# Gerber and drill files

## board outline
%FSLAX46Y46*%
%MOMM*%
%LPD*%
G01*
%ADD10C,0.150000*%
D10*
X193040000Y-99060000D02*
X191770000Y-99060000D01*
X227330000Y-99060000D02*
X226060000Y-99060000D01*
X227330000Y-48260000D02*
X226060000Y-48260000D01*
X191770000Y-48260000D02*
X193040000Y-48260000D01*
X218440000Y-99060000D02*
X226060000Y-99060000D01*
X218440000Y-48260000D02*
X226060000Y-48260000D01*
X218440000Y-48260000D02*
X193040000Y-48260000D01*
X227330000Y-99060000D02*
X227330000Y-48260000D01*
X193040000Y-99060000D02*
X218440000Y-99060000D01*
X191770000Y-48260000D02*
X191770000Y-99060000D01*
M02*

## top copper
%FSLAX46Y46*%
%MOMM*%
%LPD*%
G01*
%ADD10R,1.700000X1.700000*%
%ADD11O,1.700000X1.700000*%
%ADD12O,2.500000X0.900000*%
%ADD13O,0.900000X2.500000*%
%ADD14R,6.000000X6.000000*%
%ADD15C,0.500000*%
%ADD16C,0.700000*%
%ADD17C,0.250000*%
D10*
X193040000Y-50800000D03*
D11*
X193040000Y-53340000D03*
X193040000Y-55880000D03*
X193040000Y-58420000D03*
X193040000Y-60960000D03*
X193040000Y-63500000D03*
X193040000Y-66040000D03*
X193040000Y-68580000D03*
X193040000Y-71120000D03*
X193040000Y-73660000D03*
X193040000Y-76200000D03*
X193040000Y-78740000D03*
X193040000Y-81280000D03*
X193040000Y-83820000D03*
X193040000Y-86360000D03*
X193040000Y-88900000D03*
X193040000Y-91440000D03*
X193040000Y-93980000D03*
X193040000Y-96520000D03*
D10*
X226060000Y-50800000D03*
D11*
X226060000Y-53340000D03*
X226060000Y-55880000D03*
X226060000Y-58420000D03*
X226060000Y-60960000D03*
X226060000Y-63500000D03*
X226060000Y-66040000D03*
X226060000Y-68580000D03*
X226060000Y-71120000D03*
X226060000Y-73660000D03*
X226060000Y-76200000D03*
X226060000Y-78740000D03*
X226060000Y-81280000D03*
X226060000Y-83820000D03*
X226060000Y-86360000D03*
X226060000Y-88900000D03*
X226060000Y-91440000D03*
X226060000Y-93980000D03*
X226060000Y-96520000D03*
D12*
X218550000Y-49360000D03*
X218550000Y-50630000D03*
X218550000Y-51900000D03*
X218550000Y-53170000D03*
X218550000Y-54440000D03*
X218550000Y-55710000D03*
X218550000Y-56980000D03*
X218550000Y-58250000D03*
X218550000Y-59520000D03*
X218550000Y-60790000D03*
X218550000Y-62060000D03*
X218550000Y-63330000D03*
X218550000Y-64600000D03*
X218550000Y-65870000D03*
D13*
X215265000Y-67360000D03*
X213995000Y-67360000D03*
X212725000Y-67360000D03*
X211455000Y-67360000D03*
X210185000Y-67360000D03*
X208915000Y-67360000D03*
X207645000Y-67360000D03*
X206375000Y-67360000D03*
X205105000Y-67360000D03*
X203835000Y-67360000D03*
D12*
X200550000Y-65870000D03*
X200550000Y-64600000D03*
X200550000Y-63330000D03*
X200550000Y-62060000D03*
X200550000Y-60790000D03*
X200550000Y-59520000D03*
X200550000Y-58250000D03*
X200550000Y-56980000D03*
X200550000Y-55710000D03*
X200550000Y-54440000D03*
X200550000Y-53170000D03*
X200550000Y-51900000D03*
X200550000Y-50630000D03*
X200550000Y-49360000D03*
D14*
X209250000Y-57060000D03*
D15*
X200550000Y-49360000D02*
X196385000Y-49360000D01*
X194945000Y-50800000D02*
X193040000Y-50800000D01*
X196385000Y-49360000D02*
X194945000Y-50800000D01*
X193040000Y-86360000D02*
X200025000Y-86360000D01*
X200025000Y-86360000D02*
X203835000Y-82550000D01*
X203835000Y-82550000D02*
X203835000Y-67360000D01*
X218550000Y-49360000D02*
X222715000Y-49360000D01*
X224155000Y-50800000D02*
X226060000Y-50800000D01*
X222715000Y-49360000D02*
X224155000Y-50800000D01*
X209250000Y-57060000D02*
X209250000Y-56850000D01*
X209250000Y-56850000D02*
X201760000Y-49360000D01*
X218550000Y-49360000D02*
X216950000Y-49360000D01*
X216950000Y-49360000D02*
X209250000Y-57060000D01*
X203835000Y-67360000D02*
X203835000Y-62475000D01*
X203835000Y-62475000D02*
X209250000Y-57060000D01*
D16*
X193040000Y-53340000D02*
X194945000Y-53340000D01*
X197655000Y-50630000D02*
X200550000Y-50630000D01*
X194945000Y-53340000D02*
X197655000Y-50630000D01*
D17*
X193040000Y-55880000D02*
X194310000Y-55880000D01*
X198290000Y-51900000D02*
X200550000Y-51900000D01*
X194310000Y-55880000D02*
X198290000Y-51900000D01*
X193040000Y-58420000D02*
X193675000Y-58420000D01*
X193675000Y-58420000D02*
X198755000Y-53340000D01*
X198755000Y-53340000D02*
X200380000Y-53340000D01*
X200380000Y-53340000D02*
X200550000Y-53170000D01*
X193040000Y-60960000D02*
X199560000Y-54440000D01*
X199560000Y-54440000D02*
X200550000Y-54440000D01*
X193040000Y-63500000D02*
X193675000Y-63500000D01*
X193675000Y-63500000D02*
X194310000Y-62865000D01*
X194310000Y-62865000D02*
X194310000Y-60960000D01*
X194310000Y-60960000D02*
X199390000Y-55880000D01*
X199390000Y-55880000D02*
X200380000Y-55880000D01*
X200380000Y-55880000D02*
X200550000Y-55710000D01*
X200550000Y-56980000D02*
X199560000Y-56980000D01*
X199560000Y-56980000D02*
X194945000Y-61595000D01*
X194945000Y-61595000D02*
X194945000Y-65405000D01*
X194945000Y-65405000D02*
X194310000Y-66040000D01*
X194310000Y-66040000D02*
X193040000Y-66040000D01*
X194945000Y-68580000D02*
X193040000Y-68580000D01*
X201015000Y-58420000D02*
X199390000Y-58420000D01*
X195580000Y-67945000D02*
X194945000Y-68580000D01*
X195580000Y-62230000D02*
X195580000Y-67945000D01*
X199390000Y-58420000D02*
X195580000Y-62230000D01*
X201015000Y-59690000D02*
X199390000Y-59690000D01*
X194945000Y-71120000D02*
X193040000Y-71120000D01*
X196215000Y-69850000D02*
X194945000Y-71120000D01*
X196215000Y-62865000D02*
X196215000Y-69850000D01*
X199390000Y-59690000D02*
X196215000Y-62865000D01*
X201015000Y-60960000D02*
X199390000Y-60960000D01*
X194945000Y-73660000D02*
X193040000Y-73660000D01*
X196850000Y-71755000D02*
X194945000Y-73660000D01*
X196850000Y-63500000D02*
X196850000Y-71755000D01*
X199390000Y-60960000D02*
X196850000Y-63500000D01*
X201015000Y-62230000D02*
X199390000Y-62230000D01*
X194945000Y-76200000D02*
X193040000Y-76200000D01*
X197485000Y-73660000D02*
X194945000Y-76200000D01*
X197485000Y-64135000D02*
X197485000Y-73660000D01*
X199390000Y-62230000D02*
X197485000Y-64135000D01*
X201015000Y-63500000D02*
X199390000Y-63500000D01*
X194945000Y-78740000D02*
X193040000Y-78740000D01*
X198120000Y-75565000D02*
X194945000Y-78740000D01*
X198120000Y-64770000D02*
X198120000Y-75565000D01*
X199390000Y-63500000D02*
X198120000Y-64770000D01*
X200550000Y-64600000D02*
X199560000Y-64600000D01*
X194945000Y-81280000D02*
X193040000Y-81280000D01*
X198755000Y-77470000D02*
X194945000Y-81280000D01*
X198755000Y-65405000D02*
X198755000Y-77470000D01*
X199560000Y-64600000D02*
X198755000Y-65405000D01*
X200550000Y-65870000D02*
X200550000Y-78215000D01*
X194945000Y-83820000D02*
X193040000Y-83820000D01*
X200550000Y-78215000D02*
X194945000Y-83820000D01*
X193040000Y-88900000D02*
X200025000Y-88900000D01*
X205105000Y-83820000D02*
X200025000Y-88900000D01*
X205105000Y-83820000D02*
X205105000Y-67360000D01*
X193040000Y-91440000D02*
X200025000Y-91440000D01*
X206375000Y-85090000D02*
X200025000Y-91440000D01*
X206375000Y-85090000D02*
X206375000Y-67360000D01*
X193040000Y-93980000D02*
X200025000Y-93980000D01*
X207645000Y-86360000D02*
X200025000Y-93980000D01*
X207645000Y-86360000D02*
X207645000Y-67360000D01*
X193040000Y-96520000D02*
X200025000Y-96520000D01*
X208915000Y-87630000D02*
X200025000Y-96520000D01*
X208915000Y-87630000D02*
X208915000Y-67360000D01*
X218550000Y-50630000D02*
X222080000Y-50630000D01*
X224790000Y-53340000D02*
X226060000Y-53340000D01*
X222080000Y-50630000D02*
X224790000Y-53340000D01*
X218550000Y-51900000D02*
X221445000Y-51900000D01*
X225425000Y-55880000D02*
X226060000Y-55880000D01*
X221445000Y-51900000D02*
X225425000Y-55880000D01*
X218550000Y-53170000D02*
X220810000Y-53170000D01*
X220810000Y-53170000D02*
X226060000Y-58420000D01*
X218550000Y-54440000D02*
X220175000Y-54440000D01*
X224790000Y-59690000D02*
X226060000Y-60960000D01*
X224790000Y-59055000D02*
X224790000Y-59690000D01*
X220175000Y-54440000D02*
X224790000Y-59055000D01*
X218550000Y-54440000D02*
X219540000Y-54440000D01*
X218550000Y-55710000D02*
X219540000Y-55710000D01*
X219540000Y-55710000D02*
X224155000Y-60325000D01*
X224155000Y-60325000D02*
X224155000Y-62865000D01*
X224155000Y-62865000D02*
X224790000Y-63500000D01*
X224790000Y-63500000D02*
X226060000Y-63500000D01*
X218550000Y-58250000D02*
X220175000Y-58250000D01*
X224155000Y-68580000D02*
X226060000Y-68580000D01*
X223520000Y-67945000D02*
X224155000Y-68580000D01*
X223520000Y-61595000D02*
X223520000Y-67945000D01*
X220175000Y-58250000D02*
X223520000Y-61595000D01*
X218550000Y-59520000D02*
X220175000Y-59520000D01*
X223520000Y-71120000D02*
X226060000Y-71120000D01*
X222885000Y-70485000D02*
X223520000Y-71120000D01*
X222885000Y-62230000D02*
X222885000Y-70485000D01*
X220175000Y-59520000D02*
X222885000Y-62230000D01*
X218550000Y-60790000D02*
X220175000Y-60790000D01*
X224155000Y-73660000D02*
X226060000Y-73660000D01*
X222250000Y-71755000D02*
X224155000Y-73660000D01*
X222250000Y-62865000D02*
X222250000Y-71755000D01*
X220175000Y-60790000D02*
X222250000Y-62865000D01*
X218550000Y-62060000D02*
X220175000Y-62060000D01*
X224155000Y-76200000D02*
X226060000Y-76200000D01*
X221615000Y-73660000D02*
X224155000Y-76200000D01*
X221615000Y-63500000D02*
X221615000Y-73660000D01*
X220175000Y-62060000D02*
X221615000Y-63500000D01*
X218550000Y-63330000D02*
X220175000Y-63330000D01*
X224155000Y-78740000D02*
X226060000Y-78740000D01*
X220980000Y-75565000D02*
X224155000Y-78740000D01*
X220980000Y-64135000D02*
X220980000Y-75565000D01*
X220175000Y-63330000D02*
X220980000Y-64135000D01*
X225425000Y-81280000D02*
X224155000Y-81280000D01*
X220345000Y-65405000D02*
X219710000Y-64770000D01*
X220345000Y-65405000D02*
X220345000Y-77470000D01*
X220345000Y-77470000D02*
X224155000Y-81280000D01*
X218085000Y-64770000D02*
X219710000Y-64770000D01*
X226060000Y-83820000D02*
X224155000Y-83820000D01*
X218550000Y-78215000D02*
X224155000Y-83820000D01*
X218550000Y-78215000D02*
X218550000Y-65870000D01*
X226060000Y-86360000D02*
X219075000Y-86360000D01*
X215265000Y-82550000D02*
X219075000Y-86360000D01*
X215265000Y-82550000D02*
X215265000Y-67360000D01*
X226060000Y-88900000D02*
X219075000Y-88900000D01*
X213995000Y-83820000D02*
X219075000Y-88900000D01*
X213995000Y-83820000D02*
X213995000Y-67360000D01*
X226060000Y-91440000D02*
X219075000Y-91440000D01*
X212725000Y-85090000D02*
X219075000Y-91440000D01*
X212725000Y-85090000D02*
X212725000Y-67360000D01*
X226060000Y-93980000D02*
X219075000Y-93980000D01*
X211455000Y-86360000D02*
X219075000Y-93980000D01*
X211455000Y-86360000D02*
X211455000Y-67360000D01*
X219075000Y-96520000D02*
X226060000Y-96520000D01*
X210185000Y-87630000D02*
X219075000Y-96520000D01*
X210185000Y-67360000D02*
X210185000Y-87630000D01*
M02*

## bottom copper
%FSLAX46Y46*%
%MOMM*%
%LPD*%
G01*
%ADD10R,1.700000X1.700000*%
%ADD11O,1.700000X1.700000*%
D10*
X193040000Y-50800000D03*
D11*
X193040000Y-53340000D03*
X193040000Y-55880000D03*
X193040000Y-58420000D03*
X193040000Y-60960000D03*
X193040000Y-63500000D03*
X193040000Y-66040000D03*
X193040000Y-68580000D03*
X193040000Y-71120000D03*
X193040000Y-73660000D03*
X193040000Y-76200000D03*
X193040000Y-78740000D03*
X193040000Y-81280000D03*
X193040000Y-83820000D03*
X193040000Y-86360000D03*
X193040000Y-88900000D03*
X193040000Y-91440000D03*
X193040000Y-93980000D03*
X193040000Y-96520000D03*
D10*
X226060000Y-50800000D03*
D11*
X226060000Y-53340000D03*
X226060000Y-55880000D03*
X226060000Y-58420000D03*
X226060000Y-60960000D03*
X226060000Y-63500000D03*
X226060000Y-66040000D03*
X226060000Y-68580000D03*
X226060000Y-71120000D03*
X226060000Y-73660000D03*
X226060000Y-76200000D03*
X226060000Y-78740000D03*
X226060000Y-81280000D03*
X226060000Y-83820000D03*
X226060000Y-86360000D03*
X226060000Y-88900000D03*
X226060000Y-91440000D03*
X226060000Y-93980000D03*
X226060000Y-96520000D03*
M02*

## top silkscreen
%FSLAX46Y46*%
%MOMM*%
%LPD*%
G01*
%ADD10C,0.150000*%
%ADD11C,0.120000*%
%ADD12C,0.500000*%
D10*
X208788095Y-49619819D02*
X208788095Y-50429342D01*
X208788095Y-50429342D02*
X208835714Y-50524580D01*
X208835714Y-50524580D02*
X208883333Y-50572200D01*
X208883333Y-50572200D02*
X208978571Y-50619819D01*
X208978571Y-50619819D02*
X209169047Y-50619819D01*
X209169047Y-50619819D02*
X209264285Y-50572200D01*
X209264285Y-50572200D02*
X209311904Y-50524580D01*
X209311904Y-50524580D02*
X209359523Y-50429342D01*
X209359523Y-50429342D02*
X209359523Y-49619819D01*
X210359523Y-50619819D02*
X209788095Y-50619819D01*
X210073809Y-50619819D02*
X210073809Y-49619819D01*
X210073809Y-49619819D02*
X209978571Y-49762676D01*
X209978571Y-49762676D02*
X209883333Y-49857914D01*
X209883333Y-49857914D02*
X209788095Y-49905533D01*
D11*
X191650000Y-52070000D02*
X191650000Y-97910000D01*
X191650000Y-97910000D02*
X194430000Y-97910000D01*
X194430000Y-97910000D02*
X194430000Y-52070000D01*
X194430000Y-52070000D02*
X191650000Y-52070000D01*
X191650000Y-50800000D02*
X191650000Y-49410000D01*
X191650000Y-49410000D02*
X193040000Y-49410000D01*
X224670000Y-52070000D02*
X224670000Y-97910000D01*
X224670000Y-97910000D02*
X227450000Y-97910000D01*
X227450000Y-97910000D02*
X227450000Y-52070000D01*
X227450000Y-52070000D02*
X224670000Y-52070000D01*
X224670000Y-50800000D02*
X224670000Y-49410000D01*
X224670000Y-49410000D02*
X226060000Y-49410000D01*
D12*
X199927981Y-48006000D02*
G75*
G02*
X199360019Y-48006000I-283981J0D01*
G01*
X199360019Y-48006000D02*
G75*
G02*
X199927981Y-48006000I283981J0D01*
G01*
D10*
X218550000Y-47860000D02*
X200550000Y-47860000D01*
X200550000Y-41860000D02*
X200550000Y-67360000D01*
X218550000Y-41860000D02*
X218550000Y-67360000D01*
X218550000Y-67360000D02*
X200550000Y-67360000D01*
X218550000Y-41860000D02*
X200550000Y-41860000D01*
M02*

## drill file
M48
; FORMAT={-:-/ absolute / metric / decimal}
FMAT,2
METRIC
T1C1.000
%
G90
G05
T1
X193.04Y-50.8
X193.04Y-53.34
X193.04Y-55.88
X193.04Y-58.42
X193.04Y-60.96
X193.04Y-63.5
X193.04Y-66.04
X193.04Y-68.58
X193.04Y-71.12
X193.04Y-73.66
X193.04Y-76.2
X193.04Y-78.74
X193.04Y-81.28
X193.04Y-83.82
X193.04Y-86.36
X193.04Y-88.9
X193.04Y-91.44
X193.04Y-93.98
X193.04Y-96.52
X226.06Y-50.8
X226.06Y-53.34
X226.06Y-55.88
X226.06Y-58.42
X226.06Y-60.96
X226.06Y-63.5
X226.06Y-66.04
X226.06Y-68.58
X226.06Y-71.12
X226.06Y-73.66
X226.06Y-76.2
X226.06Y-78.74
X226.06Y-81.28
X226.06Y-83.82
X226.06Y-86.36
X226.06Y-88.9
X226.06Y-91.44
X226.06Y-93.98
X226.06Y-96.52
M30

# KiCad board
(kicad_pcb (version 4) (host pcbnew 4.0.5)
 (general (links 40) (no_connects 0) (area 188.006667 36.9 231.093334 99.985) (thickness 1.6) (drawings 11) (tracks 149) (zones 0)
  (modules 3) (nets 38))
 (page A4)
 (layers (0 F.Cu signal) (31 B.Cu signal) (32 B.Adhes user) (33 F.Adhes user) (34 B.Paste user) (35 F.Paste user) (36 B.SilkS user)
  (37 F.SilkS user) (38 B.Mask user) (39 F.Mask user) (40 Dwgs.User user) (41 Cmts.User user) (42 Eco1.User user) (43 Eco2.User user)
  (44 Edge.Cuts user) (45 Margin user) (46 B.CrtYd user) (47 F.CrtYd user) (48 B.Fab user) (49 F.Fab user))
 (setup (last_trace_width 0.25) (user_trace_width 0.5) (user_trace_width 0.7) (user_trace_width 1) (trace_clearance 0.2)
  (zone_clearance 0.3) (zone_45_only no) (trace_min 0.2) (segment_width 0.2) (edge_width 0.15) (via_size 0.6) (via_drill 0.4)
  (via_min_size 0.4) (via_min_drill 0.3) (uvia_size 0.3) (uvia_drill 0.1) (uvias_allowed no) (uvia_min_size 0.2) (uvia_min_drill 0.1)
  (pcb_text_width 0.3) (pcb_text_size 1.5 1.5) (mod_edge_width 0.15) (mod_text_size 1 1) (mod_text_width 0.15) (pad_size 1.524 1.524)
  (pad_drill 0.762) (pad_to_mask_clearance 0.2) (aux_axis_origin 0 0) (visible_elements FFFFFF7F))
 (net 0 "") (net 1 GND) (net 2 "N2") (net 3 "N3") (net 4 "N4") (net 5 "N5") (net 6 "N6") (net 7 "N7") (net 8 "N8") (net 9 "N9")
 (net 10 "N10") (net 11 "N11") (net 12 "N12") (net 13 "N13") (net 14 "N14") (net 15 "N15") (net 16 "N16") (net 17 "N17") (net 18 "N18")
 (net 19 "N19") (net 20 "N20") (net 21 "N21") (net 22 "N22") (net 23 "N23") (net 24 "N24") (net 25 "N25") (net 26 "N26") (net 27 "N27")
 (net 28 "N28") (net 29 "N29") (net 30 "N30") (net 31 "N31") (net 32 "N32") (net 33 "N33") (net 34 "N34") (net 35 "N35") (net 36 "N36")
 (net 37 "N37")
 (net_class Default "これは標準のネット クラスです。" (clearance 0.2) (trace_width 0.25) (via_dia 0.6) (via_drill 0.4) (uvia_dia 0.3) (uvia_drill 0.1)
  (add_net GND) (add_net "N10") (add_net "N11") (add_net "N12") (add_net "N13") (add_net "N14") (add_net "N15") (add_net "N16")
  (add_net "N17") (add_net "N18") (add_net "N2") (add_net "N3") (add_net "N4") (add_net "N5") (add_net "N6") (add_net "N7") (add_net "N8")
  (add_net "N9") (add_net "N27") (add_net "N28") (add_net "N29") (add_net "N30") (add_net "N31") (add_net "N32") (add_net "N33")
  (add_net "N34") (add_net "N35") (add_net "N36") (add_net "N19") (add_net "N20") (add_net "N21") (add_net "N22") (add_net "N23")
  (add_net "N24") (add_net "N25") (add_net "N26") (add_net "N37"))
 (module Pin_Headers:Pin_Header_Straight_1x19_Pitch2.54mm (layer F.Cu) (at 193.04 50.8)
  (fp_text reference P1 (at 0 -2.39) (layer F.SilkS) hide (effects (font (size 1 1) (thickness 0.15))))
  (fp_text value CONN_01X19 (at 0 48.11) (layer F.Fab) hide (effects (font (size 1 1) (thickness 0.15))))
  (fp_line (start -1.39 1.27) (end -1.39 47.11) (layer F.SilkS) (width 0.12))
  (fp_line (start -1.39 47.11) (end 1.39 47.11) (layer F.SilkS) (width 0.12))
  (fp_line (start 1.39 47.11) (end 1.39 1.27) (layer F.SilkS) (width 0.12))
  (fp_line (start 1.39 1.27) (end -1.39 1.27) (layer F.SilkS) (width 0.12))
  (fp_line (start -1.39 0) (end -1.39 -1.39) (layer F.SilkS) (width 0.12))
  (fp_line (start -1.39 -1.39) (end 0 -1.39) (layer F.SilkS) (width 0.12))
  (pad 1 thru_hole rect (at 0 0) (size 1.7 1.7) (drill 1) (layers *.Cu *.Mask) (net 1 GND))
  (pad 2 thru_hole oval (at 0 2.54) (size 1.7 1.7) (drill 1) (layers *.Cu *.Mask) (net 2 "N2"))
  (pad 3 thru_hole oval (at 0 5.08) (size 1.7 1.7) (drill 1) (layers *.Cu *.Mask) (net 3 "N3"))
  (pad 4 thru_hole oval (at 0 7.62) (size 1.7 1.7) (drill 1) (layers *.Cu *.Mask) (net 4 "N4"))
  (pad 5 thru_hole oval (at 0 10.16) (size 1.7 1.7) (drill 1) (layers *.Cu *.Mask) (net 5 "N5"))
  (pad 6 thru_hole oval (at 0 12.7) (size 1.7 1.7) (drill 1) (layers *.Cu *.Mask) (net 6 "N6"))
  (pad 7 thru_hole oval (at 0 15.24) (size 1.7 1.7) (drill 1) (layers *.Cu *.Mask) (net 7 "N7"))
  (pad 8 thru_hole oval (at 0 17.78) (size 1.7 1.7) (drill 1) (layers *.Cu *.Mask) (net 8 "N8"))
  (pad 9 thru_hole oval (at 0 20.32) (size 1.7 1.7) (drill 1) (layers *.Cu *.Mask) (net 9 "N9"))
  (pad 10 thru_hole oval (at 0 22.86) (size 1.7 1.7) (drill 1) (layers *.Cu *.Mask) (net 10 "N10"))
  (pad 11 thru_hole oval (at 0 25.4) (size 1.7 1.7) (drill 1) (layers *.Cu *.Mask) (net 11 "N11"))
  (pad 12 thru_hole oval (at 0 27.94) (size 1.7 1.7) (drill 1) (layers *.Cu *.Mask) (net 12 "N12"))
  (pad 13 thru_hole oval (at 0 30.48) (size 1.7 1.7) (drill 1) (layers *.Cu *.Mask) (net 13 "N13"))
  (pad 14 thru_hole oval (at 0 33.02) (size 1.7 1.7) (drill 1) (layers *.Cu *.Mask) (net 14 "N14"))
  (pad 15 thru_hole oval (at 0 35.56) (size 1.7 1.7) (drill 1) (layers *.Cu *.Mask) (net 1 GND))
  (pad 16 thru_hole oval (at 0 38.1) (size 1.7 1.7) (drill 1) (layers *.Cu *.Mask) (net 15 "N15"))
  (pad 17 thru_hole oval (at 0 40.64) (size 1.7 1.7) (drill 1) (layers *.Cu *.Mask) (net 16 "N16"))
  (pad 18 thru_hole oval (at 0 43.18) (size 1.7 1.7) (drill 1) (layers *.Cu *.Mask) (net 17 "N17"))
  (pad 19 thru_hole oval (at 0 45.72) (size 1.7 1.7) (drill 1) (layers *.Cu *.Mask) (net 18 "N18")))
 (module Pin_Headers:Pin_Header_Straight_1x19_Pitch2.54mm (layer F.Cu) (at 226.06 50.8)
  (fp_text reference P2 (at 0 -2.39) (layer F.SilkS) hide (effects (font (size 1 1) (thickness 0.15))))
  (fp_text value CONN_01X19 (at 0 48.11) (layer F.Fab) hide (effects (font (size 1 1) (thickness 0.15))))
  (fp_line (start -1.39 1.27) (end -1.39 47.11) (layer F.SilkS) (width 0.12))
  (fp_line (start -1.39 47.11) (end 1.39 47.11) (layer F.SilkS) (width 0.12))
  (fp_line (start 1.39 47.11) (end 1.39 1.27) (layer F.SilkS) (width 0.12))
  (fp_line (start 1.39 1.27) (end -1.39 1.27) (layer F.SilkS) (width 0.12))
  (fp_line (start -1.39 0) (end -1.39 -1.39) (layer F.SilkS) (width 0.12))
  (fp_line (start -1.39 -1.39) (end 0 -1.39) (layer F.SilkS) (width 0.12))
  (pad 1 thru_hole rect (at 0 0) (size 1.7 1.7) (drill 1) (layers *.Cu *.Mask) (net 1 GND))
  (pad 2 thru_hole oval (at 0 2.54) (size 1.7 1.7) (drill 1) (layers *.Cu *.Mask) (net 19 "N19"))
  (pad 3 thru_hole oval (at 0 5.08) (size 1.7 1.7) (drill 1) (layers *.Cu *.Mask) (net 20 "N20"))
  (pad 4 thru_hole oval (at 0 7.62) (size 1.7 1.7) (drill 1) (layers *.Cu *.Mask) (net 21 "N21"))
  (pad 5 thru_hole oval (at 0 10.16) (size 1.7 1.7) (drill 1) (layers *.Cu *.Mask) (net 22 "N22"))
  (pad 6 thru_hole oval (at 0 12.7) (size 1.7 1.7) (drill 1) (layers *.Cu *.Mask) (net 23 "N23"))
  (pad 7 thru_hole oval (at 0 15.24) (size 1.7 1.7) (drill 1) (layers *.Cu *.Mask) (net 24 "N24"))
  (pad 8 thru_hole oval (at 0 17.78) (size 1.7 1.7) (drill 1) (layers *.Cu *.Mask) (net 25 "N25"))
  (pad 9 thru_hole oval (at 0 20.32) (size 1.7 1.7) (drill 1) (layers *.Cu *.Mask) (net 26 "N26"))
  (pad 10 thru_hole oval (at 0 22.86) (size 1.7 1.7) (drill 1) (layers *.Cu *.Mask) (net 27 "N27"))
  (pad 11 thru_hole oval (at 0 25.4) (size 1.7 1.7) (drill 1) (layers *.Cu *.Mask) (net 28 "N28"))
  (pad 12 thru_hole oval (at 0 27.94) (size 1.7 1.7) (drill 1) (layers *.Cu *.Mask) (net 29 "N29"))
  (pad 13 thru_hole oval (at 0 30.48) (size 1.7 1.7) (drill 1) (layers *.Cu *.Mask) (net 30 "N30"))
  (pad 14 thru_hole oval (at 0 33.02) (size 1.7 1.7) (drill 1) (layers *.Cu *.Mask) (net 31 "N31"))
  (pad 15 thru_hole oval (at 0 35.56) (size 1.7 1.7) (drill 1) (layers *.Cu *.Mask) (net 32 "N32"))
  (pad 16 thru_hole oval (at 0 38.1) (size 1.7 1.7) (drill 1) (layers *.Cu *.Mask) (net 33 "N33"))
  (pad 17 thru_hole oval (at 0 40.64) (size 1.7 1.7) (drill 1) (layers *.Cu *.Mask) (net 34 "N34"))
  (pad 18 thru_hole oval (at 0 43.18) (size 1.7 1.7) (drill 1) (layers *.Cu *.Mask) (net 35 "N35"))
  (pad 19 thru_hole oval (at 0 45.72) (size 1.7 1.7) (drill 1) (layers *.Cu *.Mask) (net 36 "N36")))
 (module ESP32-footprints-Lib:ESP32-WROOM (layer F.Cu) (at 209.55 54.61 180)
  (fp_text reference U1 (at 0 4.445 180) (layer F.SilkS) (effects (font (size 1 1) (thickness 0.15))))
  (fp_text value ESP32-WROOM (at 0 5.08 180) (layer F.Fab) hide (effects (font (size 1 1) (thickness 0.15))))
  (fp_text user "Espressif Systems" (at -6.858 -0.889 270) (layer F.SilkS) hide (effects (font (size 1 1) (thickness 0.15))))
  (fp_circle (center 9.906 6.604) (end 10.033 6.858) (layer F.SilkS) (width 0.5))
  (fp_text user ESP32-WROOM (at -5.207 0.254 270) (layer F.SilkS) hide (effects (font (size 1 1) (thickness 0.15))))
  (fp_line (start -9 6.75) (end 9 6.75) (layer F.SilkS) (width 0.15))
  (fp_line (start 9 12.75) (end 9 -12.75) (layer F.SilkS) (width 0.15))
  (fp_line (start -9 12.75) (end -9 -12.75) (layer F.SilkS) (width 0.15))
  (fp_line (start -9 -12.75) (end 9 -12.75) (layer F.SilkS) (width 0.15))
  (fp_line (start -9 12.75) (end 9 12.75) (layer F.SilkS) (width 0.15))
  (pad 38 smd oval (at -9 5.25 180) (size 2.5 0.9) (layers F.Cu F.Paste F.Mask) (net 1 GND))
  (pad 37 smd oval (at -9 3.98 180) (size 2.5 0.9) (layers F.Cu F.Paste F.Mask) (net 19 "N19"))
  (pad 36 smd oval (at -9 2.71 180) (size 2.5 0.9) (layers F.Cu F.Paste F.Mask) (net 20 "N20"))
  (pad 35 smd oval (at -9 1.44 180) (size 2.5 0.9) (layers F.Cu F.Paste F.Mask) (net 21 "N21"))
  (pad 34 smd oval (at -9 0.17 180) (size 2.5 0.9) (layers F.Cu F.Paste F.Mask) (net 22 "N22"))
  (pad 33 smd oval (at -9 -1.1 180) (size 2.5 0.9) (layers F.Cu F.Paste F.Mask) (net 23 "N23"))
  (pad 32 smd oval (at -9 -2.37 180) (size 2.5 0.9) (layers F.Cu F.Paste F.Mask) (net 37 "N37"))
  (pad 31 smd oval (at -9 -3.64 180) (size 2.5 0.9) (layers F.Cu F.Paste F.Mask) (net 25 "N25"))
  (pad 30 smd oval (at -9 -4.91 180) (size 2.5 0.9) (layers F.Cu F.Paste F.Mask) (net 26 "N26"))
  (pad 29 smd oval (at -9 -6.18 180) (size 2.5 0.9) (layers F.Cu F.Paste F.Mask) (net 27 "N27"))
  (pad 28 smd oval (at -9 -7.45 180) (size 2.5 0.9) (layers F.Cu F.Paste F.Mask) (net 28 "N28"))
  (pad 27 smd oval (at -9 -8.72 180) (size 2.5 0.9) (layers F.Cu F.Paste F.Mask) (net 29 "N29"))
  (pad 26 smd oval (at -9 -9.99 180) (size 2.5 0.9) (layers F.Cu F.Paste F.Mask) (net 30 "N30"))
  (pad 25 smd oval (at -9 -11.26 180) (size 2.5 0.9) (layers F.Cu F.Paste F.Mask) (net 31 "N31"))
  (pad 24 smd oval (at -5.715 -12.75 180) (size 0.9 2.5) (layers F.Cu F.Paste F.Mask) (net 32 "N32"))
  (pad 23 smd oval (at -4.445 -12.75 180) (size 0.9 2.5) (layers F.Cu F.Paste F.Mask) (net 33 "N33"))
  (pad 22 smd oval (at -3.175 -12.75 180) (size 0.9 2.5) (layers F.Cu F.Paste F.Mask) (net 34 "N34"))
  (pad 21 smd oval (at -1.905 -12.75 180) (size 0.9 2.5) (layers F.Cu F.Paste F.Mask) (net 35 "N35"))
  (pad 20 smd oval (at -0.635 -12.75 180) (size 0.9 2.5) (layers F.Cu F.Paste F.Mask) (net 36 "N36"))
  (pad 19 smd oval (at 0.635 -12.75 180) (size 0.9 2.5) (layers F.Cu F.Paste F.Mask) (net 18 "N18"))
  (pad 18 smd oval (at 1.905 -12.75 180) (size 0.9 2.5) (layers F.Cu F.Paste F.Mask) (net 17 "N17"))
  (pad 17 smd oval (at 3.175 -12.75 180) (size 0.9 2.5) (layers F.Cu F.Paste F.Mask) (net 16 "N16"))
  (pad 16 smd oval (at 4.445 -12.75 180) (size 0.9 2.5) (layers F.Cu F.Paste F.Mask) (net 15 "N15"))
  (pad 15 smd oval (at 5.715 -12.75 180) (size 0.9 2.5) (layers F.Cu F.Paste F.Mask) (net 1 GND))
  (pad 14 smd oval (at 9 -11.26 180) (size 2.5 0.9) (layers F.Cu F.Paste F.Mask) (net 14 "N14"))
  (pad 13 smd oval (at 9 -9.99 180) (size 2.5 0.9) (layers F.Cu F.Paste F.Mask) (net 13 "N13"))
  (pad 12 smd oval (at 9 -8.72 180) (size 2.5 0.9) (layers F.Cu F.Paste F.Mask) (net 12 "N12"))
  (pad 11 smd oval (at 9 -7.45 180) (size 2.5 0.9) (layers F.Cu F.Paste F.Mask) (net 11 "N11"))
  (pad 10 smd oval (at 9 -6.18 180) (size 2.5 0.9) (layers F.Cu F.Paste F.Mask) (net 10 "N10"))
  (pad 9 smd oval (at 9 -4.91 180) (size 2.5 0.9) (layers F.Cu F.Paste F.Mask) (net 9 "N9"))
  (pad 8 smd oval (at 9 -3.64 180) (size 2.5 0.9) (layers F.Cu F.Paste F.Mask) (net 8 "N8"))
  (pad 7 smd oval (at 9 -2.37 180) (size 2.5 0.9) (layers F.Cu F.Paste F.Mask) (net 7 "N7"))
  (pad 6 smd oval (at 9 -1.1 180) (size 2.5 0.9) (layers F.Cu F.Paste F.Mask) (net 6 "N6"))
  (pad 5 smd oval (at 9 0.17 180) (size 2.5 0.9) (layers F.Cu F.Paste F.Mask) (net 5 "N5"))
  (pad 4 smd oval (at 9 1.44 180) (size 2.5 0.9) (layers F.Cu F.Paste F.Mask) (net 4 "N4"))
  (pad 3 smd oval (at 9 2.71 180) (size 2.5 0.9) (layers F.Cu F.Paste F.Mask) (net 3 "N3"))
  (pad 2 smd oval (at 9 3.98 180) (size 2.5 0.9) (layers F.Cu F.Paste F.Mask) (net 2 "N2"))
  (pad 1 smd oval (at 9 5.25 180) (size 2.5 0.9) (layers F.Cu F.Paste F.Mask) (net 1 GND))
  (pad 39 smd rect (at 0.3 -2.45 180) (size 6 6) (layers F.Cu F.Paste F.Mask) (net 1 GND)))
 (gr_line (start 193.04 99.06) (end 191.77 99.06) (angle 90) (layer Edge.Cuts) (width 0.15))
 (gr_line (start 227.33 99.06) (end 226.06 99.06) (angle 90) (layer Edge.Cuts) (width 0.15))
 (gr_line (start 227.33 48.26) (end 226.06 48.26) (angle 90) (layer Edge.Cuts) (width 0.15))
 (gr_line (start 191.77 48.26) (end 193.04 48.26) (angle 90) (layer Edge.Cuts) (width 0.15))
 (gr_line (start 218.44 99.06) (end 226.06 99.06) (angle 90) (layer Edge.Cuts) (width 0.15))
 (gr_line (start 218.44 48.26) (end 226.06 48.26) (angle 90) (layer Edge.Cuts) (width 0.15))
 (gr_line (start 218.44 48.26) (end 193.04 48.26) (angle 90) (layer Edge.Cuts) (width 0.15))
 (gr_line (start 227.33 99.06) (end 227.33 48.26) (angle 90) (layer Edge.Cuts) (width 0.15))
 (gr_line (start 193.04 99.06) (end 218.44 99.06) (angle 90) (layer Edge.Cuts) (width 0.15))
 (gr_line (start 191.77 48.26) (end 191.77 99.06) (angle 90) (layer Edge.Cuts) (width 0.15))
 (segment (start 200.55 49.36) (end 196.385 49.36) (width 0.5) (layer F.Cu) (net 1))
 (segment (start 194.945 50.8) (end 193.04 50.8) (width 0.5) (layer F.Cu) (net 1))
 (segment (start 196.385 49.36) (end 194.945 50.8) (width 0.5) (layer F.Cu) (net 1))
 (segment (start 193.04 86.36) (end 200.025 86.36) (width 0.5) (layer F.Cu) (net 1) (status 10))
 (segment (start 200.025 86.36) (end 203.835 82.55) (width 0.5) (layer F.Cu) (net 1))
 (segment (start 203.835 82.55) (end 203.835 67.36) (width 0.5) (layer F.Cu) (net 1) (status 20))
 (segment (start 218.55 49.36) (end 222.715 49.36) (width 0.5) (layer F.Cu) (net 1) (status 10))
 (segment (start 224.155 50.8) (end 226.06 50.8) (width 0.5) (layer F.Cu) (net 1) (status 20))
 (segment (start 222.715 49.36) (end 224.155 50.8) (width 0.5) (layer F.Cu) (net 1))
 (segment (start 209.25 57.06) (end 209.25 56.85) (width 0.5) (layer F.Cu) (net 1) (status 30))
 (segment (start 209.25 56.85) (end 201.76 49.36) (width 0.5) (layer F.Cu) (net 1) (status 30))
 (segment (start 218.55 49.36) (end 216.95 49.36) (width 0.5) (layer F.Cu) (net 1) (status 10))
 (segment (start 216.95 49.36) (end 209.25 57.06) (width 0.5) (layer F.Cu) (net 1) (status 20))
 (segment (start 203.835 67.36) (end 203.835 62.475) (width 0.5) (layer F.Cu) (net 1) (status 10))
 (segment (start 203.835 62.475) (end 209.25 57.06) (width 0.5) (layer F.Cu) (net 1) (status 20))
 (segment (start 193.04 53.34) (end 194.945 53.34) (width 0.7) (layer F.Cu) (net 2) (status 10))
 (segment (start 197.655 50.63) (end 200.55 50.63) (width 0.7) (layer F.Cu) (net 2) (status 20))
 (segment (start 194.945 53.34) (end 197.655 50.63) (width 0.7) (layer F.Cu) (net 2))
 (segment (start 193.04 55.88) (end 194.31 55.88) (width 0.25) (layer F.Cu) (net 3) (status 10))
 (segment (start 198.29 51.9) (end 200.55 51.9) (width 0.25) (layer F.Cu) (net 3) (status 20))
 (segment (start 194.31 55.88) (end 198.29 51.9) (width 0.25) (layer F.Cu) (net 3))
 (segment (start 193.04 58.42) (end 193.675 58.42) (width 0.25) (layer F.Cu) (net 4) (status 30))
 (segment (start 193.675 58.42) (end 198.755 53.34) (width 0.25) (layer F.Cu) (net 4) (status 10))
 (segment (start 198.755 53.34) (end 200.38 53.34) (width 0.25) (layer F.Cu) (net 4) (status 20))
 (segment (start 200.38 53.34) (end 200.55 53.17) (width 0.25) (layer F.Cu) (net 4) (status 30))
 (segment (start 193.04 60.96) (end 199.56 54.44) (width 0.25) (layer F.Cu) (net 5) (status 30))
 (segment (start 199.56 54.44) (end 200.55 54.44) (width 0.25) (layer F.Cu) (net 5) (status 30))
 (segment (start 193.04 63.5) (end 193.675 63.5) (width 0.25) (layer F.Cu) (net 6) (status 30))
 (segment (start 193.675 63.5) (end 194.31 62.865) (width 0.25) (layer F.Cu) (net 6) (status 10))
 (segment (start 194.31 62.865) (end 194.31 60.96) (width 0.25) (layer F.Cu) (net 6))
 (segment (start 194.31 60.96) (end 199.39 55.88) (width 0.25) (layer F.Cu) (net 6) (status 20))
 (segment (start 199.39 55.88) (end 200.38 55.88) (width 0.25) (layer F.Cu) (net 6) (status 30))
 (segment (start 200.38 55.88) (end 200.55 55.71) (width 0.25) (layer F.Cu) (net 6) (status 30))
 (segment (start 200.55 56.98) (end 199.56 56.98) (width 0.25) (layer F.Cu) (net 7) (status 30))
 (segment (start 199.56 56.98) (end 194.945 61.595) (width 0.25) (layer F.Cu) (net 7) (status 10))
 (segment (start 194.945 61.595) (end 194.945 65.405) (width 0.25) (layer F.Cu) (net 7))
 (segment (start 194.945 65.405) (end 194.31 66.04) (width 0.25) (layer F.Cu) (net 7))
 (segment (start 194.31 66.04) (end 193.04 66.04) (width 0.25) (layer F.Cu) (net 7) (status 20))
 (segment (start 194.945 68.58) (end 193.04 68.58) (width 0.25) (layer F.Cu) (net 8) (status 20))
 (segment (start 201.015 58.42) (end 199.39 58.42) (width 0.25) (layer F.Cu) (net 8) (status 30))
 (segment (start 195.58 67.945) (end 194.945 68.58) (width 0.25) (layer F.Cu) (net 8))
 (segment (start 195.58 62.23) (end 195.58 67.945) (width 0.25) (layer F.Cu) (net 8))
 (segment (start 199.39 58.42) (end 195.58 62.23) (width 0.25) (layer F.Cu) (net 8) (status 10))
 (segment (start 201.015 59.69) (end 199.39 59.69) (width 0.25) (layer F.Cu) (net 9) (status 30))
 (segment (start 194.945 71.12) (end 193.04 71.12) (width 0.25) (layer F.Cu) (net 9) (status 20))
 (segment (start 196.215 69.85) (end 194.945 71.12) (width 0.25) (layer F.Cu) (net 9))
 (segment (start 196.215 62.865) (end 196.215 69.85) (width 0.25) (layer F.Cu) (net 9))
 (segment (start 199.39 59.69) (end 196.215 62.865) (width 0.25) (layer F.Cu) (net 9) (status 10))
 (segment (start 201.015 60.96) (end 199.39 60.96) (width 0.25) (layer F.Cu) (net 10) (status 30))
 (segment (start 194.945 73.66) (end 193.04 73.66) (width 0.25) (layer F.Cu) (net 10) (status 20))
 (segment (start 196.85 71.755) (end 194.945 73.66) (width 0.25) (layer F.Cu) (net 10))
 (segment (start 196.85 63.5) (end 196.85 71.755) (width 0.25) (layer F.Cu) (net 10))
 (segment (start 199.39 60.96) (end 196.85 63.5) (width 0.25) (layer F.Cu) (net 10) (status 10))
 (segment (start 201.015 62.23) (end 199.39 62.23) (width 0.25) (layer F.Cu) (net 11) (status 30))
 (segment (start 194.945 76.2) (end 193.04 76.2) (width 0.25) (layer F.Cu) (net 11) (status 20))
 (segment (start 197.485 73.66) (end 194.945 76.2) (width 0.25) (layer F.Cu) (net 11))
 (segment (start 197.485 64.135) (end 197.485 73.66) (width 0.25) (layer F.Cu) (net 11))
 (segment (start 199.39 62.23) (end 197.485 64.135) (width 0.25) (layer F.Cu) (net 11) (status 10))
 (segment (start 201.015 63.5) (end 199.39 63.5) (width 0.25) (layer F.Cu) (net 12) (status 30))
 (segment (start 194.945 78.74) (end 193.04 78.74) (width 0.25) (layer F.Cu) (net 12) (status 20))
 (segment (start 198.12 75.565) (end 194.945 78.74) (width 0.25) (layer F.Cu) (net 12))
 (segment (start 198.12 64.77) (end 198.12 75.565) (width 0.25) (layer F.Cu) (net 12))
 (segment (start 199.39 63.5) (end 198.12 64.77) (width 0.25) (layer F.Cu) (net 12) (status 10))
 (segment (start 200.55 64.6) (end 199.56 64.6) (width 0.25) (layer F.Cu) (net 13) (status 30))
 (segment (start 194.945 81.28) (end 193.04 81.28) (width 0.25) (layer F.Cu) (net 13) (status 20))
 (segment (start 198.755 77.47) (end 194.945 81.28) (width 0.25) (layer F.Cu) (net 13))
 (segment (start 198.755 65.405) (end 198.755 77.47) (width 0.25) (layer F.Cu) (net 13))
 (segment (start 199.56 64.6) (end 198.755 65.405) (width 0.25) (layer F.Cu) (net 13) (status 10))
 (segment (start 200.55 65.87) (end 200.55 78.215) (width 0.25) (layer F.Cu) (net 14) (status 10))
 (segment (start 194.945 83.82) (end 193.04 83.82) (width 0.25) (layer F.Cu) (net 14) (status 20))
 (segment (start 200.55 78.215) (end 194.945 83.82) (width 0.25) (layer F.Cu) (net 14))
 (segment (start 193.04 88.9) (end 200.025 88.9) (width 0.25) (layer F.Cu) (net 15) (status 10))
 (segment (start 205.105 83.82) (end 200.025 88.9) (width 0.25) (layer F.Cu) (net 15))
 (segment (start 205.105 83.82) (end 205.105 67.36) (width 0.25) (layer F.Cu) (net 15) (status 20))
 (segment (start 193.04 91.44) (end 200.025 91.44) (width 0.25) (layer F.Cu) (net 16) (status 10))
 (segment (start 206.375 85.09) (end 200.025 91.44) (width 0.25) (layer F.Cu) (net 16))
 (segment (start 206.375 85.09) (end 206.375 67.36) (width 0.25) (layer F.Cu) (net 16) (status 20))
 (segment (start 193.04 93.98) (end 200.025 93.98) (width 0.25) (layer F.Cu) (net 17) (status 10))
 (segment (start 207.645 86.36) (end 200.025 93.98) (width 0.25) (layer F.Cu) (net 17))
 (segment (start 207.645 86.36) (end 207.645 67.36) (width 0.25) (layer F.Cu) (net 17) (status 20))
 (segment (start 193.04 96.52) (end 200.025 96.52) (width 0.25) (layer F.Cu) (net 18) (status 10))
 (segment (start 208.915 87.63) (end 200.025 96.52) (width 0.25) (layer F.Cu) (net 18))
 (segment (start 208.915 87.63) (end 208.915 67.36) (width 0.25) (layer F.Cu) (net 18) (status 20))
 (segment (start 218.55 50.63) (end 222.08 50.63) (width 0.25) (layer F.Cu) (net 19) (status 10))
 (segment (start 224.79 53.34) (end 226.06 53.34) (width 0.25) (layer F.Cu) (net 19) (status 20))
 (segment (start 222.08 50.63) (end 224.79 53.34) (width 0.25) (layer F.Cu) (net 19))
 (segment (start 218.55 51.9) (end 221.445 51.9) (width 0.25) (layer F.Cu) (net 20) (status 10))
 (segment (start 225.425 55.88) (end 226.06 55.88) (width 0.25) (layer F.Cu) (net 20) (status 30))
 (segment (start 221.445 51.9) (end 225.425 55.88) (width 0.25) (layer F.Cu) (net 20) (status 20))
 (segment (start 218.55 53.17) (end 220.81 53.17) (width 0.25) (layer F.Cu) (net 21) (status 10))
 (segment (start 220.81 53.17) (end 226.06 58.42) (width 0.25) (layer F.Cu) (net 21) (status 20))
 (segment (start 218.55 54.44) (end 220.175 54.44) (width 0.25) (layer F.Cu) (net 22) (status 10))
 (segment (start 224.79 59.69) (end 226.06 60.96) (width 0.25) (layer F.Cu) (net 22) (status 20))
 (segment (start 224.79 59.055) (end 224.79 59.69) (width 0.25) (layer F.Cu) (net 22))
 (segment (start 220.175 54.44) (end 224.79 59.055) (width 0.25) (layer F.Cu) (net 22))
 (segment (start 218.55 54.44) (end 219.54 54.44) (width 0.25) (layer F.Cu) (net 22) (status 30))
 (segment (start 218.55 55.71) (end 219.54 55.71) (width 0.25) (layer F.Cu) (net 23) (status 30))
 (segment (start 219.54 55.71) (end 224.155 60.325) (width 0.25) (layer F.Cu) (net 23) (status 10))
 (segment (start 224.155 60.325) (end 224.155 62.865) (width 0.25) (layer F.Cu) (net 23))
 (segment (start 224.155 62.865) (end 224.79 63.5) (width 0.25) (layer F.Cu) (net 23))
 (segment (start 224.79 63.5) (end 226.06 63.5) (width 0.25) (layer F.Cu) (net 23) (status 20))
 (segment (start 218.55 58.25) (end 220.175 58.25) (width 0.25) (layer F.Cu) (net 25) (status 10))
 (segment (start 224.155 68.58) (end 226.06 68.58) (width 0.25) (layer F.Cu) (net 25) (status 20))
 (segment (start 223.52 67.945) (end 224.155 68.58) (width 0.25) (layer F.Cu) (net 25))
 (segment (start 223.52 61.595) (end 223.52 67.945) (width 0.25) (layer F.Cu) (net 25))
 (segment (start 220.175 58.25) (end 223.52 61.595) (width 0.25) (layer F.Cu) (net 25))
 (segment (start 218.55 59.52) (end 220.175 59.52) (width 0.25) (layer F.Cu) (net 26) (status 10))
 (segment (start 223.52 71.12) (end 226.06 71.12) (width 0.25) (layer F.Cu) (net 26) (status 20))
 (segment (start 222.885 70.485) (end 223.52 71.12) (width 0.25) (layer F.Cu) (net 26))
 (segment (start 222.885 62.23) (end 222.885 70.485) (width 0.25) (layer F.Cu) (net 26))
 (segment (start 220.175 59.52) (end 222.885 62.23) (width 0.25) (layer F.Cu) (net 26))
 (segment (start 218.55 60.79) (end 220.175 60.79) (width 0.25) (layer F.Cu) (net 27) (status 10))
 (segment (start 224.155 73.66) (end 226.06 73.66) (width 0.25) (layer F.Cu) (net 27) (status 20))
 (segment (start 222.25 71.755) (end 224.155 73.66) (width 0.25) (layer F.Cu) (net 27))
 (segment (start 222.25 62.865) (end 222.25 71.755) (width 0.25) (layer F.Cu) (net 27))
 (segment (start 220.175 60.79) (end 222.25 62.865) (width 0.25) (layer F.Cu) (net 27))
 (segment (start 218.55 62.06) (end 220.175 62.06) (width 0.25) (layer F.Cu) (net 28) (status 10))
 (segment (start 224.155 76.2) (end 226.06 76.2) (width 0.25) (layer F.Cu) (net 28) (status 20))
 (segment (start 221.615 73.66) (end 224.155 76.2) (width 0.25) (layer F.Cu) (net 28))
 (segment (start 221.615 63.5) (end 221.615 73.66) (width 0.25) (layer F.Cu) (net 28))
 (segment (start 220.175 62.06) (end 221.615 63.5) (width 0.25) (layer F.Cu) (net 28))
 (segment (start 218.55 63.33) (end 220.175 63.33) (width 0.25) (layer F.Cu) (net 29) (status 10))
 (segment (start 224.155 78.74) (end 226.06 78.74) (width 0.25) (layer F.Cu) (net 29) (status 20))
 (segment (start 220.98 75.565) (end 224.155 78.74) (width 0.25) (layer F.Cu) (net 29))
 (segment (start 220.98 64.135) (end 220.98 75.565) (width 0.25) (layer F.Cu) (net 29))
 (segment (start 220.175 63.33) (end 220.98 64.135) (width 0.25) (layer F.Cu) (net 29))
 (segment (start 225.425 81.28) (end 224.155 81.28) (width 0.25) (layer F.Cu) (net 30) (status 10))
 (segment (start 220.345 65.405) (end 219.71 64.77) (width 0.25) (layer F.Cu) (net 30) (status 20))
 (segment (start 220.345 65.405) (end 220.345 77.47) (width 0.25) (layer F.Cu) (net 30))
 (segment (start 220.345 77.47) (end 224.155 81.28) (width 0.25) (layer F.Cu) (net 30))
 (segment (start 218.085 64.77) (end 219.71 64.77) (width 0.25) (layer F.Cu) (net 30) (status 30))
 (segment (start 226.06 83.82) (end 224.155 83.82) (width 0.25) (layer F.Cu) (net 31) (status 10))
 (segment (start 218.55 78.215) (end 224.155 83.82) (width 0.25) (layer F.Cu) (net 31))
 (segment (start 218.55 78.215) (end 218.55 65.87) (width 0.25) (layer F.Cu) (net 31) (status 20))
 (segment (start 226.06 86.36) (end 219.075 86.36) (width 0.25) (layer F.Cu) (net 32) (status 10))
 (segment (start 215.265 82.55) (end 219.075 86.36) (width 0.25) (layer F.Cu) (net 32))
 (segment (start 215.265 82.55) (end 215.265 67.36) (width 0.25) (layer F.Cu) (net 32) (status 20))
 (segment (start 226.06 88.9) (end 219.075 88.9) (width 0.25) (layer F.Cu) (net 33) (status 10))
 (segment (start 213.995 83.82) (end 219.075 88.9) (width 0.25) (layer F.Cu) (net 33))
 (segment (start 213.995 83.82) (end 213.995 67.36) (width 0.25) (layer F.Cu) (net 33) (status 20))
 (segment (start 226.06 91.44) (end 219.075 91.44) (width 0.25) (layer F.Cu) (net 34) (status 10))
 (segment (start 212.725 85.09) (end 219.075 91.44) (width 0.25) (layer F.Cu) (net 34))
 (segment (start 212.725 85.09) (end 212.725 67.36) (width 0.25) (layer F.Cu) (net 34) (status 20))
 (segment (start 226.06 93.98) (end 219.075 93.98) (width 0.25) (layer F.Cu) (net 35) (status 10))
 (segment (start 211.455 86.36) (end 219.075 93.98) (width 0.25) (layer F.Cu) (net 35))
 (segment (start 211.455 86.36) (end 211.455 67.36) (width 0.25) (layer F.Cu) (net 35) (status 20))
 (segment (start 219.075 96.52) (end 226.06 96.52) (width 0.25) (layer F.Cu) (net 36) (status 20))
 (segment (start 210.185 87.63) (end 219.075 96.52) (width 0.25) (layer F.Cu) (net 36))
 (segment (start 210.185 67.36) (end 210.185 87.63) (width 0.25) (layer F.Cu) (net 36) (status 10)))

